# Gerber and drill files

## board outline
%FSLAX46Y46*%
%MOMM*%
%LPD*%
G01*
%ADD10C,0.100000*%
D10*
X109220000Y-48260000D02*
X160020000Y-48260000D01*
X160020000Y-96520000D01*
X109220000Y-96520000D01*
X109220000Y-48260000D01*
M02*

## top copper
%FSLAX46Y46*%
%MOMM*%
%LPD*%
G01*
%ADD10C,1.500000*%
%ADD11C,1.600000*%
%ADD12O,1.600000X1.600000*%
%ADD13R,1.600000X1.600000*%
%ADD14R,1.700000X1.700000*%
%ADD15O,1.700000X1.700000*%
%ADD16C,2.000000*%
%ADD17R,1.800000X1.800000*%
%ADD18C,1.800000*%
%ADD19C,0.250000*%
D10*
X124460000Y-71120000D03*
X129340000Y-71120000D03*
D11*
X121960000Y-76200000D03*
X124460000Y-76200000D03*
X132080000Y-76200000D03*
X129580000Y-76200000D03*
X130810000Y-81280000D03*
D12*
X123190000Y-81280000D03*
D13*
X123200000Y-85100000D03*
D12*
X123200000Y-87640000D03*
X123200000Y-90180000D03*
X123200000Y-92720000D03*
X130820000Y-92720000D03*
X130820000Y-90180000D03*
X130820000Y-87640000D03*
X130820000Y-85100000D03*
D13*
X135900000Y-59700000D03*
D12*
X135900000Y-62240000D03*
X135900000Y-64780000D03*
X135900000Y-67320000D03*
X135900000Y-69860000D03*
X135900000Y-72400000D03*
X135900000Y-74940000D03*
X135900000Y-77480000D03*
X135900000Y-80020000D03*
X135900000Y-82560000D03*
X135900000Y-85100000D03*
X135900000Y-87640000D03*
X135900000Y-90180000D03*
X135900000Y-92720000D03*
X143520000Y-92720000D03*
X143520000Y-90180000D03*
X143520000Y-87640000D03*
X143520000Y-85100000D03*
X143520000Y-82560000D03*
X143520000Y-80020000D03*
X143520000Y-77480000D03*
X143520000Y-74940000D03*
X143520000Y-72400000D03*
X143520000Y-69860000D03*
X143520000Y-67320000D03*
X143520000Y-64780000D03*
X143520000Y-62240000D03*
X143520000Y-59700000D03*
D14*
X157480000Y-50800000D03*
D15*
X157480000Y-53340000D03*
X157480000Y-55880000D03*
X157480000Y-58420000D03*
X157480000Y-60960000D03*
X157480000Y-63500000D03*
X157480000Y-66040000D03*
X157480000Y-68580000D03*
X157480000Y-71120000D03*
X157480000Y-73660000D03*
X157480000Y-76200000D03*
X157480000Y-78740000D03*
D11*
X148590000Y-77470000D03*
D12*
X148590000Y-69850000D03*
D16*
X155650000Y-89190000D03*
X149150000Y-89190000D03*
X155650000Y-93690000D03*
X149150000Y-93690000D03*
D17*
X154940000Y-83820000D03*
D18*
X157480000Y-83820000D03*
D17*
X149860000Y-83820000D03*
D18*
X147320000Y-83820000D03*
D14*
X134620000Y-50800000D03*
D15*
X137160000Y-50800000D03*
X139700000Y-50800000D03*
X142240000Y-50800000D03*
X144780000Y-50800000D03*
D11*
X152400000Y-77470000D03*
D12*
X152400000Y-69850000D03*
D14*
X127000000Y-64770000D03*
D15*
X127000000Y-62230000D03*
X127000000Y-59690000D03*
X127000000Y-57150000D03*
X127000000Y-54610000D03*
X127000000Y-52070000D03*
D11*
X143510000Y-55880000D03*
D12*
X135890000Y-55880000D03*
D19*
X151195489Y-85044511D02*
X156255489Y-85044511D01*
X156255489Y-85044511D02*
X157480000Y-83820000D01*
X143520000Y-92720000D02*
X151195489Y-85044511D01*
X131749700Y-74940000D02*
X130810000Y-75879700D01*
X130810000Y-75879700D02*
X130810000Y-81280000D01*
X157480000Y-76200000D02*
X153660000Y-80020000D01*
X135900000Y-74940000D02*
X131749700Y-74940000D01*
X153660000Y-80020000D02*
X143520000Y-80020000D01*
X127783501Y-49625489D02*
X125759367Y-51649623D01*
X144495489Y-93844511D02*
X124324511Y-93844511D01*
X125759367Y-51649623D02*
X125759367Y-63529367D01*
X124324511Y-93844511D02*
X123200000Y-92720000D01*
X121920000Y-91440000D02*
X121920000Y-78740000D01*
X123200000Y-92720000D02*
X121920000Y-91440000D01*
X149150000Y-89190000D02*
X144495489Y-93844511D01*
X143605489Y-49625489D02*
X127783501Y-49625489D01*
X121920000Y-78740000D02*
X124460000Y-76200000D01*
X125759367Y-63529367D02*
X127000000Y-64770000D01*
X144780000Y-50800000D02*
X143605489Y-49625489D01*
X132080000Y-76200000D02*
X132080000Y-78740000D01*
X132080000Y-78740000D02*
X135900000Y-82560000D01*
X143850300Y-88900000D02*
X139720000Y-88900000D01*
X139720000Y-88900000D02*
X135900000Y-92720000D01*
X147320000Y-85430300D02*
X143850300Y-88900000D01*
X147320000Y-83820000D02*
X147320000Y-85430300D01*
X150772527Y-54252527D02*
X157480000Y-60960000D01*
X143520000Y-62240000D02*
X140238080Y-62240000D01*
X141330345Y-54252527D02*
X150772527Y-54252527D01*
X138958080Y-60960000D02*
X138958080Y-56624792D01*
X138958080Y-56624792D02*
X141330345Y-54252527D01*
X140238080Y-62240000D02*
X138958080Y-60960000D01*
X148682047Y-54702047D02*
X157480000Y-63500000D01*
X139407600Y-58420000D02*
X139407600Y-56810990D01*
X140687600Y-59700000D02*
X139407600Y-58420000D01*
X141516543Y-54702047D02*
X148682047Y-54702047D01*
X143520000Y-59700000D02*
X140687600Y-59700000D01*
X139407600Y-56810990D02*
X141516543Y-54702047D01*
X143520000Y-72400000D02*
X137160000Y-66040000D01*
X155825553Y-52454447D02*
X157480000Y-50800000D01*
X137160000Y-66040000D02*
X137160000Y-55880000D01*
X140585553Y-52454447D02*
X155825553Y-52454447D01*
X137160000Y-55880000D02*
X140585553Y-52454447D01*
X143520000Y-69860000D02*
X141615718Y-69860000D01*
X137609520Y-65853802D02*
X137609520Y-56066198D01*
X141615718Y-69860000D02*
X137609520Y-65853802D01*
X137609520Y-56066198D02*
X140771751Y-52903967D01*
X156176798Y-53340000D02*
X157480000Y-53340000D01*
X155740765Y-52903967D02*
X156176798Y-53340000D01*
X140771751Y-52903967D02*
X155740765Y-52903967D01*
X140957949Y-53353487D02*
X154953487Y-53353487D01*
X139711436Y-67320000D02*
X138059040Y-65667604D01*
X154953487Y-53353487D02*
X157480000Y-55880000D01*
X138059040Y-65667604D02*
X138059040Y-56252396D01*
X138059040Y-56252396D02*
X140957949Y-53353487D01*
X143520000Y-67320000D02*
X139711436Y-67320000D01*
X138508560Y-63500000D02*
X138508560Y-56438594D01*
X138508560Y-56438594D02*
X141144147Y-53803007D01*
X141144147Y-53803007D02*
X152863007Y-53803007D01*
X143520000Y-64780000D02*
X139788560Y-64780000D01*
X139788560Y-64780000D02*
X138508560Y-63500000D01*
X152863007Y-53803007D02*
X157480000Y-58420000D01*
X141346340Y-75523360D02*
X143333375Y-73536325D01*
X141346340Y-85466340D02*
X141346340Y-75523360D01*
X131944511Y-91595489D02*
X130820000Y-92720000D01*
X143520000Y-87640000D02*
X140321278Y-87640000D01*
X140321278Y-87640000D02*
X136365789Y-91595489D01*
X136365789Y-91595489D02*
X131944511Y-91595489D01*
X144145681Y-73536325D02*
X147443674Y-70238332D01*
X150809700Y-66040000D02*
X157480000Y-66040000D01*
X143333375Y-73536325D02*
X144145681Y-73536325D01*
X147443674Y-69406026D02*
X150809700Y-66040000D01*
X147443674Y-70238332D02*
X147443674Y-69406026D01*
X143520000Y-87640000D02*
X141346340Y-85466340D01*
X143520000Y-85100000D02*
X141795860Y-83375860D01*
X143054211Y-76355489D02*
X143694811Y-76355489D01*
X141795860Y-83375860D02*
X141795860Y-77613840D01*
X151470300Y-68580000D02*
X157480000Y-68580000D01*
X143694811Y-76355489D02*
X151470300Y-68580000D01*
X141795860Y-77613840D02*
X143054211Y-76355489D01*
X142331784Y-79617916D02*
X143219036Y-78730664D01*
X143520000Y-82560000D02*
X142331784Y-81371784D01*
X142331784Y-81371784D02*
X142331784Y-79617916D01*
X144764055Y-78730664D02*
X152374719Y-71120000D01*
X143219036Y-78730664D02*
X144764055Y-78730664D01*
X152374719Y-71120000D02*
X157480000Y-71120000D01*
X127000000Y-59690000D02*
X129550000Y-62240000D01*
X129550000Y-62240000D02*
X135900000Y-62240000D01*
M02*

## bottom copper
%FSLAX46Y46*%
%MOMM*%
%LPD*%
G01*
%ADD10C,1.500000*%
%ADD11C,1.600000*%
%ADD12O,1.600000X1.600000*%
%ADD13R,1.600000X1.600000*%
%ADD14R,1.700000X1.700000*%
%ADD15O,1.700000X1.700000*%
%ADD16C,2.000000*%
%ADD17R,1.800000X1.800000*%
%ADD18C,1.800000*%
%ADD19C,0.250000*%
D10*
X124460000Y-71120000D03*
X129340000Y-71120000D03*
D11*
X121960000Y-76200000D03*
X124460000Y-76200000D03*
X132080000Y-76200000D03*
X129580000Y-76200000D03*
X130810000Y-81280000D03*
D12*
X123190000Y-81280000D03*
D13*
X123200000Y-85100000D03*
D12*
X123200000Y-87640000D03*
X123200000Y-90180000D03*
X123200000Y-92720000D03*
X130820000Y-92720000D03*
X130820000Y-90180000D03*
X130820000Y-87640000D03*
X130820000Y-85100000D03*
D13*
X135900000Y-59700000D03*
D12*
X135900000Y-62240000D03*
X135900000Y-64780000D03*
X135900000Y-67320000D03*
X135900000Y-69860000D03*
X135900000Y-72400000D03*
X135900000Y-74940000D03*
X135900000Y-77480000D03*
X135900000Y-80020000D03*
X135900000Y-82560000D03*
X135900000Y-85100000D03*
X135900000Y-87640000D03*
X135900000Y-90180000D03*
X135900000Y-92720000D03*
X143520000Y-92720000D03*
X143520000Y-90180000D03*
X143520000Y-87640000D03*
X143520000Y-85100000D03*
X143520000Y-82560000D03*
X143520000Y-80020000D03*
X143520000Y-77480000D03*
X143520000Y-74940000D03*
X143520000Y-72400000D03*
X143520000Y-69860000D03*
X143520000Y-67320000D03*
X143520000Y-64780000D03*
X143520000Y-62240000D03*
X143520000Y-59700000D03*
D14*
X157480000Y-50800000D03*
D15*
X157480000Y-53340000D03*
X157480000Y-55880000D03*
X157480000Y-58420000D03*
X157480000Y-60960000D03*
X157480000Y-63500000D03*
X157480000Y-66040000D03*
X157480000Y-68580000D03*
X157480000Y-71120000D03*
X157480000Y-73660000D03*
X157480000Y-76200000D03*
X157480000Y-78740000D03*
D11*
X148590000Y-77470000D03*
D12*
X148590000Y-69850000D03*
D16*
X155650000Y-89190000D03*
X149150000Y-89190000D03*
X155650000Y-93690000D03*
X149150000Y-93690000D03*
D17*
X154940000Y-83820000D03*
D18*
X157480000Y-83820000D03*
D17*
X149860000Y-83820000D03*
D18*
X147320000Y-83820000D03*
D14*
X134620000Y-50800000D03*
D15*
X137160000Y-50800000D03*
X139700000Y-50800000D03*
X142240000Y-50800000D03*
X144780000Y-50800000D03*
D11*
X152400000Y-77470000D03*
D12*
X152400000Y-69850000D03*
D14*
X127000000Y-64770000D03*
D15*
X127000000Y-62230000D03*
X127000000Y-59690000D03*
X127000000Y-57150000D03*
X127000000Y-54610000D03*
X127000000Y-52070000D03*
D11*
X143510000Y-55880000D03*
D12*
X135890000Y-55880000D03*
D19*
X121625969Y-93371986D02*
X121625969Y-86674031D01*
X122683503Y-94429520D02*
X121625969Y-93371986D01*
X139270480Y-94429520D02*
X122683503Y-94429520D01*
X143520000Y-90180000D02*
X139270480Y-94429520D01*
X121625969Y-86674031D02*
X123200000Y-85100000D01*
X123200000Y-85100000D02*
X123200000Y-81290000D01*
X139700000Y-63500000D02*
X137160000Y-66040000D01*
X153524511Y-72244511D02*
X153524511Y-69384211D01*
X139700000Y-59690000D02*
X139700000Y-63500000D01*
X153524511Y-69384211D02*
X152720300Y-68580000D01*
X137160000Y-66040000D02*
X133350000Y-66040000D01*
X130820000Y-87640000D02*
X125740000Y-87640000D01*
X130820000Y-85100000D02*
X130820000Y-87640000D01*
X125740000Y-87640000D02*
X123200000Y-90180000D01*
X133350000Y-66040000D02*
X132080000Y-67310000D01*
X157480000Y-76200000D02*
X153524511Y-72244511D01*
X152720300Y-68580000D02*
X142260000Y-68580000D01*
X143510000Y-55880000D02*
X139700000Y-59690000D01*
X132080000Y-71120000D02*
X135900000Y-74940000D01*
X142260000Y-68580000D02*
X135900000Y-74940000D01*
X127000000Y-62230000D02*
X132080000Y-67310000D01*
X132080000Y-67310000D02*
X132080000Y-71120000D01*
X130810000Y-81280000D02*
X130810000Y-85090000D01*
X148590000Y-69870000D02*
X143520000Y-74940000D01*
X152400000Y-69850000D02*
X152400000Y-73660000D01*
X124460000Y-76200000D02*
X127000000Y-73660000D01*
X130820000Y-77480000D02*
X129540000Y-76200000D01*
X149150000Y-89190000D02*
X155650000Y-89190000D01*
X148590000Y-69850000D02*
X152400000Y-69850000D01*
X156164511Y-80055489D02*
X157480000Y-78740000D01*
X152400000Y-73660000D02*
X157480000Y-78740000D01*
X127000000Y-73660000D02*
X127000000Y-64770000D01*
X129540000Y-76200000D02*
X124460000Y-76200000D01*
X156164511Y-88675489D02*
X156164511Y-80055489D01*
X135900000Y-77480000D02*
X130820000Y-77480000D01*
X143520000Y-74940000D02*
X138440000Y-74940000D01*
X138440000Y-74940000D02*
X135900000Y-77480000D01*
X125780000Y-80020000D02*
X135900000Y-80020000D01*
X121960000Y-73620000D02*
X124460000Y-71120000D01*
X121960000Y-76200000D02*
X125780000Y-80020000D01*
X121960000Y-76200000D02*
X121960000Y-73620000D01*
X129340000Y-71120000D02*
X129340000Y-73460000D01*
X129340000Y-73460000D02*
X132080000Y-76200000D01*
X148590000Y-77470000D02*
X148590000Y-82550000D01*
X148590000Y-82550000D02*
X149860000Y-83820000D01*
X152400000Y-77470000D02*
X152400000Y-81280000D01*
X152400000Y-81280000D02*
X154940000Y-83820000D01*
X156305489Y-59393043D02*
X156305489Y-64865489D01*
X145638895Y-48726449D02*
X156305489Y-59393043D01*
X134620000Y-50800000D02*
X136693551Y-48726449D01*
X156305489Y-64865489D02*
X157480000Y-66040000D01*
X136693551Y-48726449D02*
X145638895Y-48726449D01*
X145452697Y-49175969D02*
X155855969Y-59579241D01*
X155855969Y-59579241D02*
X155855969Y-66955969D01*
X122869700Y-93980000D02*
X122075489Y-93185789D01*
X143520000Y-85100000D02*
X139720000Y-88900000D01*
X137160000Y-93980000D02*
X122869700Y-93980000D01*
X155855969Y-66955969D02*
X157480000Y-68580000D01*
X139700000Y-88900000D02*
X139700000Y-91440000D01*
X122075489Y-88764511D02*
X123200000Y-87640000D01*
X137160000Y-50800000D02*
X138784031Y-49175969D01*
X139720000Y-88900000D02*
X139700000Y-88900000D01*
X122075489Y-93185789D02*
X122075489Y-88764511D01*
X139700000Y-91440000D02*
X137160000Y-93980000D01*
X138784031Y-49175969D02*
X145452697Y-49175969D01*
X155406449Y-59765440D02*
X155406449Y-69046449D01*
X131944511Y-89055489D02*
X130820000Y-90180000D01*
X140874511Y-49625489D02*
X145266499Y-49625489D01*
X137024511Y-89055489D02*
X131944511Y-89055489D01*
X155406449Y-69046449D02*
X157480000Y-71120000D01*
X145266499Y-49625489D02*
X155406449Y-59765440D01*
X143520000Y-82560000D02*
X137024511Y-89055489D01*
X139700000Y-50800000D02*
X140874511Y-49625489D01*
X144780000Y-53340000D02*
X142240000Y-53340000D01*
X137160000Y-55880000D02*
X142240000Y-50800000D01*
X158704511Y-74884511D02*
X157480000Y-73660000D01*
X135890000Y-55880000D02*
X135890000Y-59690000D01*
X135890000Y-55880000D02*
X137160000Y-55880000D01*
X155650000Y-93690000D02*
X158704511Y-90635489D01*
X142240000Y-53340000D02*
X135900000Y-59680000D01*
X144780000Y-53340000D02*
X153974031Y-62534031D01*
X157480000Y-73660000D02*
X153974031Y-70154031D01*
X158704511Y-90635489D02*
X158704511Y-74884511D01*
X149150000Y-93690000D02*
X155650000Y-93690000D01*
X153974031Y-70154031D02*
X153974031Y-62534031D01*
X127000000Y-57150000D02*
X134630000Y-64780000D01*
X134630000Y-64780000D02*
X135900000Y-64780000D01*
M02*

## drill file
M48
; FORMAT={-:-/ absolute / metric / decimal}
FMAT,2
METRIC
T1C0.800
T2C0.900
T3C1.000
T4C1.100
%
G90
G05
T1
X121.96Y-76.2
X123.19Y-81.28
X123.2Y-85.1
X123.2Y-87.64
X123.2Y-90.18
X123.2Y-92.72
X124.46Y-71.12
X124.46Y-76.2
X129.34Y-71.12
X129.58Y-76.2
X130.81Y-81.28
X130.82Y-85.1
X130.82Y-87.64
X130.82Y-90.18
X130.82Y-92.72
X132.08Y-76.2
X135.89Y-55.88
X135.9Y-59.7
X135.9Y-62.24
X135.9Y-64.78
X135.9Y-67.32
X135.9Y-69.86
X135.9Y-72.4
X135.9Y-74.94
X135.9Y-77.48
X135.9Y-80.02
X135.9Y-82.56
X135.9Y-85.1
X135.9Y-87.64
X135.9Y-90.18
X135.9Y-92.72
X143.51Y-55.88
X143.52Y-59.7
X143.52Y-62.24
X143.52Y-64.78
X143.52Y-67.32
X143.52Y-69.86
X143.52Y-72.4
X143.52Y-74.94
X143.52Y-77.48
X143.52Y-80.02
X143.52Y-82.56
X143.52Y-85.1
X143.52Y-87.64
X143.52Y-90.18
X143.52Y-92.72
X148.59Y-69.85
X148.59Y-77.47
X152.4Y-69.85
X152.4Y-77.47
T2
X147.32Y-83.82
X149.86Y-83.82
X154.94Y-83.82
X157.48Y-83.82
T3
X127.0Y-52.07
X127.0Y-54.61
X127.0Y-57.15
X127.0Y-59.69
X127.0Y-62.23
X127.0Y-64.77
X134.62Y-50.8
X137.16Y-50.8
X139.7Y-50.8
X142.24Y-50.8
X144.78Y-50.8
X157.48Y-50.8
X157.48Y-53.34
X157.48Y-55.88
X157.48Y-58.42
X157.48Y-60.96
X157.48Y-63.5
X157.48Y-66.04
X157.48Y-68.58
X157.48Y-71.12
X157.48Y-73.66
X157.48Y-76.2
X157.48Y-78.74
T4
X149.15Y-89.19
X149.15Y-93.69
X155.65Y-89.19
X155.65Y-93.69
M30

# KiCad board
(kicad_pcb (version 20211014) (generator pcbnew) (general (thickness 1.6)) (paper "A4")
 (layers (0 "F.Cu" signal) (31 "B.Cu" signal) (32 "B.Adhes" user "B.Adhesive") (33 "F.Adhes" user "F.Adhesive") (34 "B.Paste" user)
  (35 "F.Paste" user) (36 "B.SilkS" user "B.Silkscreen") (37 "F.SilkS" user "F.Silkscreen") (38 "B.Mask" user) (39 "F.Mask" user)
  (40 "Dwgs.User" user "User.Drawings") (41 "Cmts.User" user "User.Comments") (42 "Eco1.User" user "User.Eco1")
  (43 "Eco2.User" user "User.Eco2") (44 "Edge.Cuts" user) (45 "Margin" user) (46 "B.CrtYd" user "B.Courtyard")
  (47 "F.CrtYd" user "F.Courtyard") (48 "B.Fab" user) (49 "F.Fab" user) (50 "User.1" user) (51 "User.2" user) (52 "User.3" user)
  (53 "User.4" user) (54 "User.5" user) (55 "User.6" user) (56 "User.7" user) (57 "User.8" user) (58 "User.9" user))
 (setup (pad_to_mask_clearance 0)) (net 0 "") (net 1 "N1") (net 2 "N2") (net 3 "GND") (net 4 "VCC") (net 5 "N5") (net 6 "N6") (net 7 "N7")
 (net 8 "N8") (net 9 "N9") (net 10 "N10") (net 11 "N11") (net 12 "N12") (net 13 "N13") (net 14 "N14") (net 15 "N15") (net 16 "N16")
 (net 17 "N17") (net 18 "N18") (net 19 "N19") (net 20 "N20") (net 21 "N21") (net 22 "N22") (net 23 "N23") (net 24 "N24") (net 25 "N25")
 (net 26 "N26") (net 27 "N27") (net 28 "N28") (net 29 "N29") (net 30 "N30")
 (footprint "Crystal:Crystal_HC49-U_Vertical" (layer "F.Cu") (at 124.46 71.12)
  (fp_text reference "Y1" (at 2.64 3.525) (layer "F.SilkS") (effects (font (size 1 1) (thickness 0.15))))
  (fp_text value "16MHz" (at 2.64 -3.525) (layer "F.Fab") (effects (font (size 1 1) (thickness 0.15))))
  (pad "1" thru_hole circle locked (at 0 0) (size 1.5 1.5) (drill 0.8) (layers *.Cu *.Mask) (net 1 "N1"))
  (pad "2" thru_hole circle locked (at 4.88 0) (size 1.5 1.5) (drill 0.8) (layers *.Cu *.Mask) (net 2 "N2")))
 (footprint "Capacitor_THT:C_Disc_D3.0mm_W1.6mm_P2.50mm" (layer "F.Cu") (at 121.96 76.2)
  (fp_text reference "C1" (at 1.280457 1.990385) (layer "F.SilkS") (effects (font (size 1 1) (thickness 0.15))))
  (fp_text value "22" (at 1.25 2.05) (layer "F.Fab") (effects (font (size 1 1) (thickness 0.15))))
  (pad "1" thru_hole circle locked (at 0 0) (size 1.6 1.6) (drill 0.8) (layers *.Cu *.Mask) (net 1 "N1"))
  (pad "2" thru_hole circle locked (at 2.5 0) (size 1.6 1.6) (drill 0.8) (layers *.Cu *.Mask) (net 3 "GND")))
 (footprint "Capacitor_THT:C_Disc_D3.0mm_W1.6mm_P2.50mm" (layer "F.Cu") (at 132.08 76.2 180)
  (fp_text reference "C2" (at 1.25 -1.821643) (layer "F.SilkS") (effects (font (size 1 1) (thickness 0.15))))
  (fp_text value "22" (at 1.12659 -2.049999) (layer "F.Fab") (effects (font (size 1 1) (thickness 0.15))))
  (pad "1" thru_hole circle locked (at 0 0 180) (size 1.6 1.6) (drill 0.8) (layers *.Cu *.Mask) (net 2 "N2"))
  (pad "2" thru_hole circle locked (at 2.5 0 180) (size 1.6 1.6) (drill 0.8) (layers *.Cu *.Mask) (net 3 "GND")))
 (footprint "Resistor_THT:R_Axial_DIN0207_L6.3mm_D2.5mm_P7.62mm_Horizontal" (layer "F.Cu") (at 130.81 81.28 180)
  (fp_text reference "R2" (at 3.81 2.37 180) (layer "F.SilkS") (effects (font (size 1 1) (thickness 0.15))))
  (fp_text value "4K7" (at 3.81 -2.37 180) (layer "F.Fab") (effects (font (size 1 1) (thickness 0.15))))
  (pad "1" thru_hole circle locked (at 0 0 180) (size 1.6 1.6) (drill 0.8) (layers *.Cu *.Mask) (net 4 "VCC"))
  (pad "2" thru_hole oval locked (at 7.62 0 180) (size 1.6 1.6) (drill 0.8) (layers *.Cu *.Mask) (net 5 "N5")))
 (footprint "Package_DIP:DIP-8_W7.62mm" (layer "F.Cu") (at 123.2 85.1)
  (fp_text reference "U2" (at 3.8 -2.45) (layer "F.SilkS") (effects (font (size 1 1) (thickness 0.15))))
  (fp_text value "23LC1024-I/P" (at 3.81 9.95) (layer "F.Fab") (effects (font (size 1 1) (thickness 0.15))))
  (pad "1" thru_hole rect locked (at 0 0) (size 1.6 1.6) (drill 0.8) (layers *.Cu *.Mask) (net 5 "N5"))
  (pad "2" thru_hole oval locked (at 0 2.54) (size 1.6 1.6) (drill 0.8) (layers *.Cu *.Mask) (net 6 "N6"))
  (pad "3" thru_hole oval locked (at 0 5.08) (size 1.6 1.6) (drill 0.8) (layers *.Cu *.Mask) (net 4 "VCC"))
  (pad "4" thru_hole oval locked (at 0 7.62) (size 1.6 1.6) (drill 0.8) (layers *.Cu *.Mask) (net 3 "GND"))
  (pad "5" thru_hole oval locked (at 7.62 7.62) (size 1.6 1.6) (drill 0.8) (layers *.Cu *.Mask) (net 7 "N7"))
  (pad "6" thru_hole oval locked (at 7.62 5.08) (size 1.6 1.6) (drill 0.8) (layers *.Cu *.Mask) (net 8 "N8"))
  (pad "7" thru_hole oval locked (at 7.62 2.54) (size 1.6 1.6) (drill 0.8) (layers *.Cu *.Mask) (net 4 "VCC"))
  (pad "8" thru_hole oval locked (at 7.62 0) (size 1.6 1.6) (drill 0.8) (layers *.Cu *.Mask) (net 4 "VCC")))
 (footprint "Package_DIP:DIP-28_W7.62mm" (layer "F.Cu") (at 135.9 59.7)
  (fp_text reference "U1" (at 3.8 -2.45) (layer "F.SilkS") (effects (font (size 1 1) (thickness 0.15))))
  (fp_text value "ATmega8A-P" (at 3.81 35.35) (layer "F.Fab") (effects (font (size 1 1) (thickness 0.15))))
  (pad "1" thru_hole rect locked (at 0 0) (size 1.6 1.6) (drill 0.8) (layers *.Cu *.Mask) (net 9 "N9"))
  (pad "2" thru_hole oval locked (at 0 2.54) (size 1.6 1.6) (drill 0.8) (layers *.Cu *.Mask) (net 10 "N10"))
  (pad "3" thru_hole oval locked (at 0 5.08) (size 1.6 1.6) (drill 0.8) (layers *.Cu *.Mask) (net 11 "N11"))
  (pad "4" thru_hole oval locked (at 0 7.62) (size 1.6 1.6) (drill 0.8) (layers *.Cu *.Mask) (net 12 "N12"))
  (pad "5" thru_hole oval locked (at 0 10.16) (size 1.6 1.6) (drill 0.8) (layers *.Cu *.Mask) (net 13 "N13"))
  (pad "6" thru_hole oval locked (at 0 12.7) (size 1.6 1.6) (drill 0.8) (layers *.Cu *.Mask) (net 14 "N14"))
  (pad "7" thru_hole oval locked (at 0 15.24) (size 1.6 1.6) (drill 0.8) (layers *.Cu *.Mask) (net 4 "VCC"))
  (pad "8" thru_hole oval locked (at 0 17.78) (size 1.6 1.6) (drill 0.8) (layers *.Cu *.Mask) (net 3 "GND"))
  (pad "9" thru_hole oval locked (at 0 20.32) (size 1.6 1.6) (drill 0.8) (layers *.Cu *.Mask) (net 1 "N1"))
  (pad "10" thru_hole oval locked (at 0 22.86) (size 1.6 1.6) (drill 0.8) (layers *.Cu *.Mask) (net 2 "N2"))
  (pad "11" thru_hole oval locked (at 0 25.4) (size 1.6 1.6) (drill 0.8) (layers *.Cu *.Mask) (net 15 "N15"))
  (pad "12" thru_hole oval locked (at 0 27.94) (size 1.6 1.6) (drill 0.8) (layers *.Cu *.Mask) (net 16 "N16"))
  (pad "13" thru_hole oval locked (at 0 30.48) (size 1.6 1.6) (drill 0.8) (layers *.Cu *.Mask) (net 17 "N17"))
  (pad "14" thru_hole oval locked (at 0 33.02) (size 1.6 1.6) (drill 0.8) (layers *.Cu *.Mask) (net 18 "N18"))
  (pad "15" thru_hole oval locked (at 7.62 33.02) (size 1.6 1.6) (drill 0.8) (layers *.Cu *.Mask) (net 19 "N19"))
  (pad "16" thru_hole oval locked (at 7.62 30.48) (size 1.6 1.6) (drill 0.8) (layers *.Cu *.Mask) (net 5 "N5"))
  (pad "17" thru_hole oval locked (at 7.62 27.94) (size 1.6 1.6) (drill 0.8) (layers *.Cu *.Mask) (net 7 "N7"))
  (pad "18" thru_hole oval locked (at 7.62 25.4) (size 1.6 1.6) (drill 0.8) (layers *.Cu *.Mask) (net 6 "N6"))
  (pad "19" thru_hole oval locked (at 7.62 22.86) (size 1.6 1.6) (drill 0.8) (layers *.Cu *.Mask) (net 8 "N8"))
  (pad "20" thru_hole oval locked (at 7.62 20.32) (size 1.6 1.6) (drill 0.8) (layers *.Cu *.Mask) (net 4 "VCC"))
  (pad "21" thru_hole oval locked (at 7.62 17.78) (size 1.6 1.6) (drill 0.8) (layers *.Cu *.Mask) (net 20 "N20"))
  (pad "22" thru_hole oval locked (at 7.62 15.24) (size 1.6 1.6) (drill 0.8) (layers *.Cu *.Mask) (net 3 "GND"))
  (pad "23" thru_hole oval locked (at 7.62 12.7) (size 1.6 1.6) (drill 0.8) (layers *.Cu *.Mask) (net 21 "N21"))
  (pad "24" thru_hole oval locked (at 7.62 10.16) (size 1.6 1.6) (drill 0.8) (layers *.Cu *.Mask) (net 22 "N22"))
  (pad "25" thru_hole oval locked (at 7.62 7.62) (size 1.6 1.6) (drill 0.8) (layers *.Cu *.Mask) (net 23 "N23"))
  (pad "26" thru_hole oval locked (at 7.62 5.08) (size 1.6 1.6) (drill 0.8) (layers *.Cu *.Mask) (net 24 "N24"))
  (pad "27" thru_hole oval locked (at 7.62 2.54) (size 1.6 1.6) (drill 0.8) (layers *.Cu *.Mask) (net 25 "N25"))
  (pad "28" thru_hole oval locked (at 7.62 0) (size 1.6 1.6) (drill 0.8) (layers *.Cu *.Mask) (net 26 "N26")))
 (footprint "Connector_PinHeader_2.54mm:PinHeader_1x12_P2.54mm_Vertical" (layer "F.Cu") (at 157.48 50.8)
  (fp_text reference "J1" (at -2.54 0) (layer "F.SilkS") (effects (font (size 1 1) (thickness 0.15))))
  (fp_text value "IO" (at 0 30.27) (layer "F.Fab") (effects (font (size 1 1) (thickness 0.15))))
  (pad "1" thru_hole rect locked (at 0 0) (size 1.7 1.7) (drill 1) (layers *.Cu *.Mask) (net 21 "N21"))
  (pad "2" thru_hole oval locked (at 0 2.54) (size 1.7 1.7) (drill 1) (layers *.Cu *.Mask) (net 22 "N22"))
  (pad "3" thru_hole oval locked (at 0 5.08) (size 1.7 1.7) (drill 1) (layers *.Cu *.Mask) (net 23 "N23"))
  (pad "4" thru_hole oval locked (at 0 7.62) (size 1.7 1.7) (drill 1) (layers *.Cu *.Mask) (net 24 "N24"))
  (pad "5" thru_hole oval locked (at 0 10.16) (size 1.7 1.7) (drill 1) (layers *.Cu *.Mask) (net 25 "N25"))
  (pad "6" thru_hole oval locked (at 0 12.7) (size 1.7 1.7) (drill 1) (layers *.Cu *.Mask) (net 26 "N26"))
  (pad "7" thru_hole oval locked (at 0 15.24) (size 1.7 1.7) (drill 1) (layers *.Cu *.Mask) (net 7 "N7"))
  (pad "8" thru_hole oval locked (at 0 17.78) (size 1.7 1.7) (drill 1) (layers *.Cu *.Mask) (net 6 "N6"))
  (pad "9" thru_hole oval locked (at 0 20.32) (size 1.7 1.7) (drill 1) (layers *.Cu *.Mask) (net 8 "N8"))
  (pad "10" thru_hole oval locked (at 0 22.86) (size 1.7 1.7) (drill 1) (layers *.Cu *.Mask) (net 9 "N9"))
  (pad "11" thru_hole oval locked (at 0 25.4) (size 1.7 1.7) (drill 1) (layers *.Cu *.Mask) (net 4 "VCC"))
  (pad "12" thru_hole oval locked (at 0 27.94) (size 1.7 1.7) (drill 1) (layers *.Cu *.Mask) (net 3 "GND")))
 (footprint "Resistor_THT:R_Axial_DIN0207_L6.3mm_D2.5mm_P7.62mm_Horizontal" (layer "F.Cu") (at 148.59 77.47 90)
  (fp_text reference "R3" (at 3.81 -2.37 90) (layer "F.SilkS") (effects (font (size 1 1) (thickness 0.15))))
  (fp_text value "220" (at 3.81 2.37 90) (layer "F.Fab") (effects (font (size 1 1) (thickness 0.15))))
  (pad "1" thru_hole circle locked (at 0 0 90) (size 1.6 1.6) (drill 0.8) (layers *.Cu *.Mask) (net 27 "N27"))
  (pad "2" thru_hole oval locked (at 7.62 0 90) (size 1.6 1.6) (drill 0.8) (layers *.Cu *.Mask) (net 3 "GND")))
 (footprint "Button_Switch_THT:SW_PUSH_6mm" (layer "F.Cu") (at 149.15 89.19)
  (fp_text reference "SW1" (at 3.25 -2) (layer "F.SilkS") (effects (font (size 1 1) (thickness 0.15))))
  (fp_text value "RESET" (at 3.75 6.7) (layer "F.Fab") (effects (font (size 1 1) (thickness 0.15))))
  (pad "1" thru_hole circle locked (at 6.5 0 90) (size 2 2) (drill 1.1) (layers *.Cu *.Mask) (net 3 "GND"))
  (pad "1" thru_hole circle locked (at 0 0 90) (size 2 2) (drill 1.1) (layers *.Cu *.Mask) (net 3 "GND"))
  (pad "2" thru_hole circle locked (at 6.5 4.5 90) (size 2 2) (drill 1.1) (layers *.Cu *.Mask) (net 9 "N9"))
  (pad "2" thru_hole circle locked (at 0 4.5 90) (size 2 2) (drill 1.1) (layers *.Cu *.Mask) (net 9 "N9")))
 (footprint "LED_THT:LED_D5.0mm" (layer "F.Cu") (at 154.94 83.82)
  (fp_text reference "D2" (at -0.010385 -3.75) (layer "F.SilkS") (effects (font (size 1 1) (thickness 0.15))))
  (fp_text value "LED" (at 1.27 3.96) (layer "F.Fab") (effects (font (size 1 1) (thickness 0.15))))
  (pad "1" thru_hole rect locked (at 0 0) (size 1.8 1.8) (drill 0.9) (layers *.Cu *.Mask) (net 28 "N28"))
  (pad "2" thru_hole circle locked (at 2.54 0) (size 1.8 1.8) (drill 0.9) (layers *.Cu *.Mask) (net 19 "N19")))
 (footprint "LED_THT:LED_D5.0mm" (layer "F.Cu") (at 149.86 83.82 180)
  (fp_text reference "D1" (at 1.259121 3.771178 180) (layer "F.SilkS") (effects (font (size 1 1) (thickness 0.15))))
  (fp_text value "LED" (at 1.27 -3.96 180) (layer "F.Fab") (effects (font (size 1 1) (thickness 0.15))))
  (pad "1" thru_hole rect locked (at 0 0 180) (size 1.8 1.8) (drill 0.9) (layers *.Cu *.Mask) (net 27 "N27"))
  (pad "2" thru_hole circle locked (at 2.54 0 180) (size 1.8 1.8) (drill 0.9) (layers *.Cu *.Mask) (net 18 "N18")))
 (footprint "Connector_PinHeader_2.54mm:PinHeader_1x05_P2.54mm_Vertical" (layer "F.Cu") (at 134.62 50.8 90)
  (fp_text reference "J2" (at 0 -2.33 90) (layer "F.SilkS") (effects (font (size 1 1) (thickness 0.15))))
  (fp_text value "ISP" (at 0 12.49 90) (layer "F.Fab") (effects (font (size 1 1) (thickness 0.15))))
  (pad "1" thru_hole rect locked (at 0 0 90) (size 1.7 1.7) (drill 1) (layers *.Cu *.Mask) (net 7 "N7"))
  (pad "2" thru_hole oval locked (at 0 2.54 90) (size 1.7 1.7) (drill 1) (layers *.Cu *.Mask) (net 6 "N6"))
  (pad "3" thru_hole oval locked (at 0 5.08 90) (size 1.7 1.7) (drill 1) (layers *.Cu *.Mask) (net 8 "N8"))
  (pad "4" thru_hole oval locked (at 0 7.62 90) (size 1.7 1.7) (drill 1) (layers *.Cu *.Mask) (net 9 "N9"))
  (pad "5" thru_hole oval locked (at 0 10.16 90) (size 1.7 1.7) (drill 1) (layers *.Cu *.Mask) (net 3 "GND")))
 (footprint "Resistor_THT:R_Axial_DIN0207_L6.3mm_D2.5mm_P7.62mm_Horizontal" (layer "F.Cu") (at 152.4 77.47 90)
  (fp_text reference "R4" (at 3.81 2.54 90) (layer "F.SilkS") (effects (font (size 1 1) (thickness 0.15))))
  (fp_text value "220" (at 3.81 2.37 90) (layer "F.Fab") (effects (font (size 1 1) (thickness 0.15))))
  (pad "1" thru_hole circle locked (at 0 0 90) (size 1.6 1.6) (drill 0.8) (layers *.Cu *.Mask) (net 28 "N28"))
  (pad "2" thru_hole oval locked (at 7.62 0 90) (size 1.6 1.6) (drill 0.8) (layers *.Cu *.Mask) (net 3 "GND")))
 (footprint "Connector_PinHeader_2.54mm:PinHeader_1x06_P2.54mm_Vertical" (layer "F.Cu") (at 127 64.77 180)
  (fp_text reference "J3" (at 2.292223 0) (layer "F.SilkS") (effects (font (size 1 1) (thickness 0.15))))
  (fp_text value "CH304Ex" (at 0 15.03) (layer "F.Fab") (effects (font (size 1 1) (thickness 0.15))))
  (pad "1" thru_hole rect locked (at 0 0 180) (size 1.7 1.7) (drill 1) (layers *.Cu *.Mask) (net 3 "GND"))
  (pad "2" thru_hole oval locked (at 0 2.54 180) (size 1.7 1.7) (drill 1) (layers *.Cu *.Mask) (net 4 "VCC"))
  (pad "3" thru_hole oval locked (at 0 5.08 180) (size 1.7 1.7) (drill 1) (layers *.Cu *.Mask) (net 10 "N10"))
  (pad "4" thru_hole oval locked (at 0 7.62 180) (size 1.7 1.7) (drill 1) (layers *.Cu *.Mask) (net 11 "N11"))
  (pad "5" thru_hole oval locked (at 0 10.16 180) (size 1.7 1.7) (drill 1) (layers *.Cu *.Mask) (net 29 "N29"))
  (pad "6" thru_hole oval locked (at 0 12.7 180) (size 1.7 1.7) (drill 1) (layers *.Cu *.Mask) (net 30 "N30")))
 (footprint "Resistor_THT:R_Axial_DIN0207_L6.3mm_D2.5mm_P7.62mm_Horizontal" (layer "F.Cu") (at 143.51 55.88 180)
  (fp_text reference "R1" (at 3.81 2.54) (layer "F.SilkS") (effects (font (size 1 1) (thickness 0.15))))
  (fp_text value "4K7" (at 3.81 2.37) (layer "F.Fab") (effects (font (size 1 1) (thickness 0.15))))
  (pad "1" thru_hole circle locked (at 0 0 180) (size 1.6 1.6) (drill 0.8) (layers *.Cu *.Mask) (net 4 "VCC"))
  (pad "2" thru_hole oval locked (at 7.62 0 180) (size 1.6 1.6) (drill 0.8) (layers *.Cu *.Mask) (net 9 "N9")))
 (gr_rect (start 109.22 48.26) (end 160.02 96.52) (layer "Edge.Cuts") (width 0.1) (fill none))
 (segment (start 151.195489 85.044511) (end 156.255489 85.044511) (width 0.25) (layer "F.Cu") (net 19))
 (segment (start 156.255489 85.044511) (end 157.48 83.82) (width 0.25) (layer "F.Cu") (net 19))
 (segment (start 143.52 92.72) (end 151.195489 85.044511) (width 0.25) (layer "F.Cu") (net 19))
 (segment (start 121.625969 93.371986) (end 121.625969 86.674031) (width 0.25) (layer "B.Cu") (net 5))
 (segment (start 122.683503 94.42952) (end 121.625969 93.371986) (width 0.25) (layer "B.Cu") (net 5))
 (segment (start 139.27048 94.42952) (end 122.683503 94.42952) (width 0.25) (layer "B.Cu") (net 5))
 (segment (start 143.52 90.18) (end 139.27048 94.42952) (width 0.25) (layer "B.Cu") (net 5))
 (segment (start 121.625969 86.674031) (end 123.2 85.1) (width 0.25) (layer "B.Cu") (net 5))
 (segment (start 123.2 85.1) (end 123.2 81.29) (width 0.25) (layer "B.Cu") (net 5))
 (segment (start 131.7497 74.94) (end 130.81 75.8797) (width 0.25) (layer "F.Cu") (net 4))
 (segment (start 130.81 75.8797) (end 130.81 81.28) (width 0.25) (layer "F.Cu") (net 4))
 (segment (start 157.48 76.2) (end 153.66 80.02) (width 0.25) (layer "F.Cu") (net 4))
 (segment (start 135.9 74.94) (end 131.7497 74.94) (width 0.25) (layer "F.Cu") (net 4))
 (segment (start 153.66 80.02) (end 143.52 80.02) (width 0.25) (layer "F.Cu") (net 4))
 (segment (start 139.7 63.5) (end 137.16 66.04) (width 0.25) (layer "B.Cu") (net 4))
 (segment (start 153.524511 72.244511) (end 153.524511 69.384211) (width 0.25) (layer "B.Cu") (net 4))
 (segment (start 139.7 59.69) (end 139.7 63.5) (width 0.25) (layer "B.Cu") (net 4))
 (segment (start 153.524511 69.384211) (end 152.7203 68.58) (width 0.25) (layer "B.Cu") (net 4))
 (segment (start 137.16 66.04) (end 133.35 66.04) (width 0.25) (layer "B.Cu") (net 4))
 (segment (start 130.82 87.64) (end 125.74 87.64) (width 0.25) (layer "B.Cu") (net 4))
 (segment (start 130.82 85.1) (end 130.82 87.64) (width 0.25) (layer "B.Cu") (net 4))
 (segment (start 125.74 87.64) (end 123.2 90.18) (width 0.25) (layer "B.Cu") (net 4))
 (segment (start 133.35 66.04) (end 132.08 67.31) (width 0.25) (layer "B.Cu") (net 4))
 (segment (start 157.48 76.2) (end 153.524511 72.244511) (width 0.25) (layer "B.Cu") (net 4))
 (segment (start 152.7203 68.58) (end 142.26 68.58) (width 0.25) (layer "B.Cu") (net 4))
 (segment (start 143.51 55.88) (end 139.7 59.69) (width 0.25) (layer "B.Cu") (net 4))
 (segment (start 132.08 71.12) (end 135.9 74.94) (width 0.25) (layer "B.Cu") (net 4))
 (segment (start 142.26 68.58) (end 135.9 74.94) (width 0.25) (layer "B.Cu") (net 4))
 (segment (start 127 62.23) (end 132.08 67.31) (width 0.25) (layer "B.Cu") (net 4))
 (segment (start 132.08 67.31) (end 132.08 71.12) (width 0.25) (layer "B.Cu") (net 4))
 (segment (start 130.81 81.28) (end 130.81 85.09) (width 0.25) (layer "B.Cu") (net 4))
 (segment (start 127.783501 49.625489) (end 125.759367 51.649623) (width 0.25) (layer "F.Cu") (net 3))
 (segment (start 144.495489 93.844511) (end 124.324511 93.844511) (width 0.25) (layer "F.Cu") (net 3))
 (segment (start 125.759367 51.649623) (end 125.759367 63.529367) (width 0.25) (layer "F.Cu") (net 3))
 (segment (start 124.324511 93.844511) (end 123.2 92.72) (width 0.25) (layer "F.Cu") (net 3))
 (segment (start 121.92 91.44) (end 121.92 78.74) (width 0.25) (layer "F.Cu") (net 3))
 (segment (start 123.2 92.72) (end 121.92 91.44) (width 0.25) (layer "F.Cu") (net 3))
 (segment (start 149.15 89.19) (end 144.495489 93.844511) (width 0.25) (layer "F.Cu") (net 3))
 (segment (start 143.605489 49.625489) (end 127.783501 49.625489) (width 0.25) (layer "F.Cu") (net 3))
 (segment (start 121.92 78.74) (end 124.46 76.2) (width 0.25) (layer "F.Cu") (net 3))
 (segment (start 125.759367 63.529367) (end 127 64.77) (width 0.25) (layer "F.Cu") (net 3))
 (segment (start 144.78 50.8) (end 143.605489 49.625489) (width 0.25) (layer "F.Cu") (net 3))
 (segment (start 148.59 69.87) (end 143.52 74.94) (width 0.25) (layer "B.Cu") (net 3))
 (segment (start 152.4 69.85) (end 152.4 73.66) (width 0.25) (layer "B.Cu") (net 3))
 (segment (start 124.46 76.2) (end 127 73.66) (width 0.25) (layer "B.Cu") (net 3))
 (segment (start 130.82 77.48) (end 129.54 76.2) (width 0.25) (layer "B.Cu") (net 3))
 (segment (start 149.15 89.19) (end 155.65 89.19) (width 0.25) (layer "B.Cu") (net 3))
 (segment (start 148.59 69.85) (end 152.4 69.85) (width 0.25) (layer "B.Cu") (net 3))
 (segment (start 156.164511 80.055489) (end 157.48 78.74) (width 0.25) (layer "B.Cu") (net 3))
 (segment (start 152.4 73.66) (end 157.48 78.74) (width 0.25) (layer "B.Cu") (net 3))
 (segment (start 127 73.66) (end 127 64.77) (width 0.25) (layer "B.Cu") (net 3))
 (segment (start 129.54 76.2) (end 124.46 76.2) (width 0.25) (layer "B.Cu") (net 3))
 (segment (start 156.164511 88.675489) (end 156.164511 80.055489) (width 0.25) (layer "B.Cu") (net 3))
 (segment (start 135.9 77.48) (end 130.82 77.48) (width 0.25) (layer "B.Cu") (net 3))
 (segment (start 143.52 74.94) (end 138.44 74.94) (width 0.25) (layer "B.Cu") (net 3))
 (segment (start 138.44 74.94) (end 135.9 77.48) (width 0.25) (layer "B.Cu") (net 3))
 (segment (start 125.78 80.02) (end 135.9 80.02) (width 0.25) (layer "B.Cu") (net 1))
 (segment (start 121.96 73.62) (end 124.46 71.12) (width 0.25) (layer "B.Cu") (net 1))
 (segment (start 121.96 76.2) (end 125.78 80.02) (width 0.25) (layer "B.Cu") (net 1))
 (segment (start 121.96 76.2) (end 121.96 73.62) (width 0.25) (layer "B.Cu") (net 1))
 (segment (start 132.08 76.2) (end 132.08 78.74) (width 0.25) (layer "F.Cu") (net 2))
 (segment (start 132.08 78.74) (end 135.9 82.56) (width 0.25) (layer "F.Cu") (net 2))
 (segment (start 129.34 71.12) (end 129.34 73.46) (width 0.25) (layer "B.Cu") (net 2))
 (segment (start 129.34 73.46) (end 132.08 76.2) (width 0.25) (layer "B.Cu") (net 2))
 (segment (start 143.8503 88.9) (end 139.72 88.9) (width 0.25) (layer "F.Cu") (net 18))
 (segment (start 139.72 88.9) (end 135.9 92.72) (width 0.25) (layer "F.Cu") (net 18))
 (segment (start 147.32 85.4303) (end 143.8503 88.9) (width 0.25) (layer "F.Cu") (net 18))
 (segment (start 147.32 83.82) (end 147.32 85.4303) (width 0.25) (layer "F.Cu") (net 18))
 (segment (start 148.59 77.47) (end 148.59 82.55) (width 0.25) (layer "B.Cu") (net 27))
 (segment (start 148.59 82.55) (end 149.86 83.82) (width 0.25) (layer "B.Cu") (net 27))
 (segment (start 152.4 77.47) (end 152.4 81.28) (width 0.25) (layer "B.Cu") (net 28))
 (segment (start 152.4 81.28) (end 154.94 83.82) (width 0.25) (layer "B.Cu") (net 28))
 (segment (start 150.772527 54.252527) (end 157.48 60.96) (width 0.25) (layer "F.Cu") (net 25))
 (segment (start 143.52 62.24) (end 140.23808 62.24) (width 0.25) (layer "F.Cu") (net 25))
 (segment (start 141.330345 54.252527) (end 150.772527 54.252527) (width 0.25) (layer "F.Cu") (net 25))
 (segment (start 138.95808 60.96) (end 138.95808 56.624792) (width 0.25) (layer "F.Cu") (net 25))
 (segment (start 138.95808 56.624792) (end 141.330345 54.252527) (width 0.25) (layer "F.Cu") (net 25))
 (segment (start 140.23808 62.24) (end 138.95808 60.96) (width 0.25) (layer "F.Cu") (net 25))
 (segment (start 148.682047 54.702047) (end 157.48 63.5) (width 0.25) (layer "F.Cu") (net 26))
 (segment (start 139.4076 58.42) (end 139.4076 56.81099) (width 0.25) (layer "F.Cu") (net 26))
 (segment (start 140.6876 59.7) (end 139.4076 58.42) (width 0.25) (layer "F.Cu") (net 26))
 (segment (start 141.516543 54.702047) (end 148.682047 54.702047) (width 0.25) (layer "F.Cu") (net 26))
 (segment (start 143.52 59.7) (end 140.6876 59.7) (width 0.25) (layer "F.Cu") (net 26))
 (segment (start 139.4076 56.81099) (end 141.516543 54.702047) (width 0.25) (layer "F.Cu") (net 26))
 (segment (start 143.52 72.4) (end 137.16 66.04) (width 0.25) (layer "F.Cu") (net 21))
 (segment (start 155.825553 52.454447) (end 157.48 50.8) (width 0.25) (layer "F.Cu") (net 21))
 (segment (start 137.16 66.04) (end 137.16 55.88) (width 0.25) (layer "F.Cu") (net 21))
 (segment (start 140.585553 52.454447) (end 155.825553 52.454447) (width 0.25) (layer "F.Cu") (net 21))
 (segment (start 137.16 55.88) (end 140.585553 52.454447) (width 0.25) (layer "F.Cu") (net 21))
 (segment (start 143.52 69.86) (end 141.615718 69.86) (width 0.25) (layer "F.Cu") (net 22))
 (segment (start 137.60952 65.853802) (end 137.60952 56.066198) (width 0.25) (layer "F.Cu") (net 22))
 (segment (start 141.615718 69.86) (end 137.60952 65.853802) (width 0.25) (layer "F.Cu") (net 22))
 (segment (start 137.60952 56.066198) (end 140.771751 52.903967) (width 0.25) (layer "F.Cu") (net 22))
 (segment (start 156.176798 53.34) (end 157.48 53.34) (width 0.25) (layer "F.Cu") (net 22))
 (segment (start 155.740765 52.903967) (end 156.176798 53.34) (width 0.25) (layer "F.Cu") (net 22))
 (segment (start 140.771751 52.903967) (end 155.740765 52.903967) (width 0.25) (layer "F.Cu") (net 22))
 (segment (start 140.957949 53.353487) (end 154.953487 53.353487) (width 0.25) (layer "F.Cu") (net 23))
 (segment (start 139.711436 67.32) (end 138.05904 65.667604) (width 0.25) (layer "F.Cu") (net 23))
 (segment (start 154.953487 53.353487) (end 157.48 55.88) (width 0.25) (layer "F.Cu") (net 23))
 (segment (start 138.05904 65.667604) (end 138.05904 56.252396) (width 0.25) (layer "F.Cu") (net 23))
 (segment (start 138.05904 56.252396) (end 140.957949 53.353487) (width 0.25) (layer "F.Cu") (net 23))
 (segment (start 143.52 67.32) (end 139.711436 67.32) (width 0.25) (layer "F.Cu") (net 23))
 (segment (start 138.50856 63.5) (end 138.50856 56.438594) (width 0.25) (layer "F.Cu") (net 24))
 (segment (start 138.50856 56.438594) (end 141.144147 53.803007) (width 0.25) (layer "F.Cu") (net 24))
 (segment (start 141.144147 53.803007) (end 152.863007 53.803007) (width 0.25) (layer "F.Cu") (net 24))
 (segment (start 143.52 64.78) (end 139.78856 64.78) (width 0.25) (layer "F.Cu") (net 24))
 (segment (start 139.78856 64.78) (end 138.50856 63.5) (width 0.25) (layer "F.Cu") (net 24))
 (segment (start 152.863007 53.803007) (end 157.48 58.42) (width 0.25) (layer "F.Cu") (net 24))
 (segment (start 141.34634 75.52336) (end 143.333375 73.536325) (width 0.25) (layer "F.Cu") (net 7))
 (segment (start 141.34634 85.46634) (end 141.34634 75.52336) (width 0.25) (layer "F.Cu") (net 7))
 (segment (start 131.944511 91.595489) (end 130.82 92.72) (width 0.25) (layer "F.Cu") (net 7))
 (segment (start 143.52 87.64) (end 140.321278 87.64) (width 0.25) (layer "F.Cu") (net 7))
 (segment (start 140.321278 87.64) (end 136.365789 91.595489) (width 0.25) (layer "F.Cu") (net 7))
 (segment (start 136.365789 91.595489) (end 131.944511 91.595489) (width 0.25) (layer "F.Cu") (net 7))
 (segment (start 144.145681 73.536325) (end 147.443674 70.238332) (width 0.25) (layer "F.Cu") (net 7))
 (segment (start 150.8097 66.04) (end 157.48 66.04) (width 0.25) (layer "F.Cu") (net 7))
 (segment (start 143.333375 73.536325) (end 144.145681 73.536325) (width 0.25) (layer "F.Cu") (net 7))
 (segment (start 147.443674 69.406026) (end 150.8097 66.04) (width 0.25) (layer "F.Cu") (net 7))
 (segment (start 147.443674 70.238332) (end 147.443674 69.406026) (width 0.25) (layer "F.Cu") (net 7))
 (segment (start 143.52 87.64) (end 141.34634 85.46634) (width 0.25) (layer "F.Cu") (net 7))
 (segment (start 156.305489 59.393043) (end 156.305489 64.865489) (width 0.25) (layer "B.Cu") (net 7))
 (segment (start 145.638895 48.726449) (end 156.305489 59.393043) (width 0.25) (layer "B.Cu") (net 7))
 (segment (start 134.62 50.8) (end 136.693551 48.726449) (width 0.25) (layer "B.Cu") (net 7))
 (segment (start 156.305489 64.865489) (end 157.48 66.04) (width 0.25) (layer "B.Cu") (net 7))
 (segment (start 136.693551 48.726449) (end 145.638895 48.726449) (width 0.25) (layer "B.Cu") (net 7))
 (segment (start 143.52 85.1) (end 141.79586 83.37586) (width 0.25) (layer "F.Cu") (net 6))
 (segment (start 143.054211 76.355489) (end 143.694811 76.355489) (width 0.25) (layer "F.Cu") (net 6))
 (segment (start 141.79586 83.37586) (end 141.79586 77.61384) (width 0.25) (layer "F.Cu") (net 6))
 (segment (start 151.4703 68.58) (end 157.48 68.58) (width 0.25) (layer "F.Cu") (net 6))
 (segment (start 143.694811 76.355489) (end 151.4703 68.58) (width 0.25) (layer "F.Cu") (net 6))
 (segment (start 141.79586 77.61384) (end 143.054211 76.355489) (width 0.25) (layer "F.Cu") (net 6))
 (segment (start 145.452697 49.175969) (end 155.855969 59.579241) (width 0.25) (layer "B.Cu") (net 6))
 (segment (start 155.855969 59.579241) (end 155.855969 66.955969) (width 0.25) (layer "B.Cu") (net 6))
 (segment (start 122.8697 93.98) (end 122.075489 93.185789) (width 0.25) (layer "B.Cu") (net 6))
 (segment (start 143.52 85.1) (end 139.72 88.9) (width 0.25) (layer "B.Cu") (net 6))
 (segment (start 137.16 93.98) (end 122.8697 93.98) (width 0.25) (layer "B.Cu") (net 6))
 (segment (start 155.855969 66.955969) (end 157.48 68.58) (width 0.25) (layer "B.Cu") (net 6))
 (segment (start 139.7 88.9) (end 139.7 91.44) (width 0.25) (layer "B.Cu") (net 6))
 (segment (start 122.075489 88.764511) (end 123.2 87.64) (width 0.25) (layer "B.Cu") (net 6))
 (segment (start 137.16 50.8) (end 138.784031 49.175969) (width 0.25) (layer "B.Cu") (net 6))
 (segment (start 139.72 88.9) (end 139.7 88.9) (width 0.25) (layer "B.Cu") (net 6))
 (segment (start 122.075489 93.185789) (end 122.075489 88.764511) (width 0.25) (layer "B.Cu") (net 6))
 (segment (start 139.7 91.44) (end 137.16 93.98) (width 0.25) (layer "B.Cu") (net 6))
 (segment (start 138.784031 49.175969) (end 145.452697 49.175969) (width 0.25) (layer "B.Cu") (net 6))
 (segment (start 142.331784 79.617916) (end 143.219036 78.730664) (width 0.25) (layer "F.Cu") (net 8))
 (segment (start 143.52 82.56) (end 142.331784 81.371784) (width 0.25) (layer "F.Cu") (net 8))
 (segment (start 142.331784 81.371784) (end 142.331784 79.617916) (width 0.25) (layer "F.Cu") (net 8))
 (segment (start 144.764055 78.730664) (end 152.374719 71.12) (width 0.25) (layer "F.Cu") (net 8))
 (segment (start 143.219036 78.730664) (end 144.764055 78.730664) (width 0.25) (layer "F.Cu") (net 8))
 (segment (start 152.374719 71.12) (end 157.48 71.12) (width 0.25) (layer "F.Cu") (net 8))
 (segment (start 155.406449 59.76544) (end 155.406449 69.046449) (width 0.25) (layer "B.Cu") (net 8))
 (segment (start 131.944511 89.055489) (end 130.82 90.18) (width 0.25) (layer "B.Cu") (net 8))
 (segment (start 140.874511 49.625489) (end 145.266499 49.625489) (width 0.25) (layer "B.Cu") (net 8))
 (segment (start 137.024511 89.055489) (end 131.944511 89.055489) (width 0.25) (layer "B.Cu") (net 8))
 (segment (start 155.406449 69.046449) (end 157.48 71.12) (width 0.25) (layer "B.Cu") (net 8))
 (segment (start 145.266499 49.625489) (end 155.406449 59.76544) (width 0.25) (layer "B.Cu") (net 8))
 (segment (start 143.52 82.56) (end 137.024511 89.055489) (width 0.25) (layer "B.Cu") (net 8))
 (segment (start 139.7 50.8) (end 140.874511 49.625489) (width 0.25) (layer "B.Cu") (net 8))
 (segment (start 144.78 53.34) (end 142.24 53.34) (width 0.25) (layer "B.Cu") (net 9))
 (segment (start 137.16 55.88) (end 142.24 50.8) (width 0.25) (layer "B.Cu") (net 9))
 (segment (start 158.704511 74.884511) (end 157.48 73.66) (width 0.25) (layer "B.Cu") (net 9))
 (segment (start 135.89 55.88) (end 135.89 59.69) (width 0.25) (layer "B.Cu") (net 9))
 (segment (start 135.89 55.88) (end 137.16 55.88) (width 0.25) (layer "B.Cu") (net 9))
 (segment (start 155.65 93.69) (end 158.704511 90.635489) (width 0.25) (layer "B.Cu") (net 9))
 (segment (start 142.24 53.34) (end 135.9 59.68) (width 0.25) (layer "B.Cu") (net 9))
 (segment (start 144.78 53.34) (end 153.974031 62.534031) (width 0.25) (layer "B.Cu") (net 9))
 (segment (start 157.48 73.66) (end 153.974031 70.154031) (width 0.25) (layer "B.Cu") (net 9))
 (segment (start 158.704511 90.635489) (end 158.704511 74.884511) (width 0.25) (layer "B.Cu") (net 9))
 (segment (start 149.15 93.69) (end 155.65 93.69) (width 0.25) (layer "B.Cu") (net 9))
 (segment (start 153.974031 70.154031) (end 153.974031 62.534031) (width 0.25) (layer "B.Cu") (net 9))
 (segment (start 127 59.69) (end 129.55 62.24) (width 0.25) (layer "F.Cu") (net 10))
 (segment (start 129.55 62.24) (end 135.9 62.24) (width 0.25) (layer "F.Cu") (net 10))
 (segment (start 127 57.15) (end 134.63 64.78) (width 0.25) (layer "B.Cu") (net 11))
 (segment (start 134.63 64.78) (end 135.9 64.78) (width 0.25) (layer "B.Cu") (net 11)))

